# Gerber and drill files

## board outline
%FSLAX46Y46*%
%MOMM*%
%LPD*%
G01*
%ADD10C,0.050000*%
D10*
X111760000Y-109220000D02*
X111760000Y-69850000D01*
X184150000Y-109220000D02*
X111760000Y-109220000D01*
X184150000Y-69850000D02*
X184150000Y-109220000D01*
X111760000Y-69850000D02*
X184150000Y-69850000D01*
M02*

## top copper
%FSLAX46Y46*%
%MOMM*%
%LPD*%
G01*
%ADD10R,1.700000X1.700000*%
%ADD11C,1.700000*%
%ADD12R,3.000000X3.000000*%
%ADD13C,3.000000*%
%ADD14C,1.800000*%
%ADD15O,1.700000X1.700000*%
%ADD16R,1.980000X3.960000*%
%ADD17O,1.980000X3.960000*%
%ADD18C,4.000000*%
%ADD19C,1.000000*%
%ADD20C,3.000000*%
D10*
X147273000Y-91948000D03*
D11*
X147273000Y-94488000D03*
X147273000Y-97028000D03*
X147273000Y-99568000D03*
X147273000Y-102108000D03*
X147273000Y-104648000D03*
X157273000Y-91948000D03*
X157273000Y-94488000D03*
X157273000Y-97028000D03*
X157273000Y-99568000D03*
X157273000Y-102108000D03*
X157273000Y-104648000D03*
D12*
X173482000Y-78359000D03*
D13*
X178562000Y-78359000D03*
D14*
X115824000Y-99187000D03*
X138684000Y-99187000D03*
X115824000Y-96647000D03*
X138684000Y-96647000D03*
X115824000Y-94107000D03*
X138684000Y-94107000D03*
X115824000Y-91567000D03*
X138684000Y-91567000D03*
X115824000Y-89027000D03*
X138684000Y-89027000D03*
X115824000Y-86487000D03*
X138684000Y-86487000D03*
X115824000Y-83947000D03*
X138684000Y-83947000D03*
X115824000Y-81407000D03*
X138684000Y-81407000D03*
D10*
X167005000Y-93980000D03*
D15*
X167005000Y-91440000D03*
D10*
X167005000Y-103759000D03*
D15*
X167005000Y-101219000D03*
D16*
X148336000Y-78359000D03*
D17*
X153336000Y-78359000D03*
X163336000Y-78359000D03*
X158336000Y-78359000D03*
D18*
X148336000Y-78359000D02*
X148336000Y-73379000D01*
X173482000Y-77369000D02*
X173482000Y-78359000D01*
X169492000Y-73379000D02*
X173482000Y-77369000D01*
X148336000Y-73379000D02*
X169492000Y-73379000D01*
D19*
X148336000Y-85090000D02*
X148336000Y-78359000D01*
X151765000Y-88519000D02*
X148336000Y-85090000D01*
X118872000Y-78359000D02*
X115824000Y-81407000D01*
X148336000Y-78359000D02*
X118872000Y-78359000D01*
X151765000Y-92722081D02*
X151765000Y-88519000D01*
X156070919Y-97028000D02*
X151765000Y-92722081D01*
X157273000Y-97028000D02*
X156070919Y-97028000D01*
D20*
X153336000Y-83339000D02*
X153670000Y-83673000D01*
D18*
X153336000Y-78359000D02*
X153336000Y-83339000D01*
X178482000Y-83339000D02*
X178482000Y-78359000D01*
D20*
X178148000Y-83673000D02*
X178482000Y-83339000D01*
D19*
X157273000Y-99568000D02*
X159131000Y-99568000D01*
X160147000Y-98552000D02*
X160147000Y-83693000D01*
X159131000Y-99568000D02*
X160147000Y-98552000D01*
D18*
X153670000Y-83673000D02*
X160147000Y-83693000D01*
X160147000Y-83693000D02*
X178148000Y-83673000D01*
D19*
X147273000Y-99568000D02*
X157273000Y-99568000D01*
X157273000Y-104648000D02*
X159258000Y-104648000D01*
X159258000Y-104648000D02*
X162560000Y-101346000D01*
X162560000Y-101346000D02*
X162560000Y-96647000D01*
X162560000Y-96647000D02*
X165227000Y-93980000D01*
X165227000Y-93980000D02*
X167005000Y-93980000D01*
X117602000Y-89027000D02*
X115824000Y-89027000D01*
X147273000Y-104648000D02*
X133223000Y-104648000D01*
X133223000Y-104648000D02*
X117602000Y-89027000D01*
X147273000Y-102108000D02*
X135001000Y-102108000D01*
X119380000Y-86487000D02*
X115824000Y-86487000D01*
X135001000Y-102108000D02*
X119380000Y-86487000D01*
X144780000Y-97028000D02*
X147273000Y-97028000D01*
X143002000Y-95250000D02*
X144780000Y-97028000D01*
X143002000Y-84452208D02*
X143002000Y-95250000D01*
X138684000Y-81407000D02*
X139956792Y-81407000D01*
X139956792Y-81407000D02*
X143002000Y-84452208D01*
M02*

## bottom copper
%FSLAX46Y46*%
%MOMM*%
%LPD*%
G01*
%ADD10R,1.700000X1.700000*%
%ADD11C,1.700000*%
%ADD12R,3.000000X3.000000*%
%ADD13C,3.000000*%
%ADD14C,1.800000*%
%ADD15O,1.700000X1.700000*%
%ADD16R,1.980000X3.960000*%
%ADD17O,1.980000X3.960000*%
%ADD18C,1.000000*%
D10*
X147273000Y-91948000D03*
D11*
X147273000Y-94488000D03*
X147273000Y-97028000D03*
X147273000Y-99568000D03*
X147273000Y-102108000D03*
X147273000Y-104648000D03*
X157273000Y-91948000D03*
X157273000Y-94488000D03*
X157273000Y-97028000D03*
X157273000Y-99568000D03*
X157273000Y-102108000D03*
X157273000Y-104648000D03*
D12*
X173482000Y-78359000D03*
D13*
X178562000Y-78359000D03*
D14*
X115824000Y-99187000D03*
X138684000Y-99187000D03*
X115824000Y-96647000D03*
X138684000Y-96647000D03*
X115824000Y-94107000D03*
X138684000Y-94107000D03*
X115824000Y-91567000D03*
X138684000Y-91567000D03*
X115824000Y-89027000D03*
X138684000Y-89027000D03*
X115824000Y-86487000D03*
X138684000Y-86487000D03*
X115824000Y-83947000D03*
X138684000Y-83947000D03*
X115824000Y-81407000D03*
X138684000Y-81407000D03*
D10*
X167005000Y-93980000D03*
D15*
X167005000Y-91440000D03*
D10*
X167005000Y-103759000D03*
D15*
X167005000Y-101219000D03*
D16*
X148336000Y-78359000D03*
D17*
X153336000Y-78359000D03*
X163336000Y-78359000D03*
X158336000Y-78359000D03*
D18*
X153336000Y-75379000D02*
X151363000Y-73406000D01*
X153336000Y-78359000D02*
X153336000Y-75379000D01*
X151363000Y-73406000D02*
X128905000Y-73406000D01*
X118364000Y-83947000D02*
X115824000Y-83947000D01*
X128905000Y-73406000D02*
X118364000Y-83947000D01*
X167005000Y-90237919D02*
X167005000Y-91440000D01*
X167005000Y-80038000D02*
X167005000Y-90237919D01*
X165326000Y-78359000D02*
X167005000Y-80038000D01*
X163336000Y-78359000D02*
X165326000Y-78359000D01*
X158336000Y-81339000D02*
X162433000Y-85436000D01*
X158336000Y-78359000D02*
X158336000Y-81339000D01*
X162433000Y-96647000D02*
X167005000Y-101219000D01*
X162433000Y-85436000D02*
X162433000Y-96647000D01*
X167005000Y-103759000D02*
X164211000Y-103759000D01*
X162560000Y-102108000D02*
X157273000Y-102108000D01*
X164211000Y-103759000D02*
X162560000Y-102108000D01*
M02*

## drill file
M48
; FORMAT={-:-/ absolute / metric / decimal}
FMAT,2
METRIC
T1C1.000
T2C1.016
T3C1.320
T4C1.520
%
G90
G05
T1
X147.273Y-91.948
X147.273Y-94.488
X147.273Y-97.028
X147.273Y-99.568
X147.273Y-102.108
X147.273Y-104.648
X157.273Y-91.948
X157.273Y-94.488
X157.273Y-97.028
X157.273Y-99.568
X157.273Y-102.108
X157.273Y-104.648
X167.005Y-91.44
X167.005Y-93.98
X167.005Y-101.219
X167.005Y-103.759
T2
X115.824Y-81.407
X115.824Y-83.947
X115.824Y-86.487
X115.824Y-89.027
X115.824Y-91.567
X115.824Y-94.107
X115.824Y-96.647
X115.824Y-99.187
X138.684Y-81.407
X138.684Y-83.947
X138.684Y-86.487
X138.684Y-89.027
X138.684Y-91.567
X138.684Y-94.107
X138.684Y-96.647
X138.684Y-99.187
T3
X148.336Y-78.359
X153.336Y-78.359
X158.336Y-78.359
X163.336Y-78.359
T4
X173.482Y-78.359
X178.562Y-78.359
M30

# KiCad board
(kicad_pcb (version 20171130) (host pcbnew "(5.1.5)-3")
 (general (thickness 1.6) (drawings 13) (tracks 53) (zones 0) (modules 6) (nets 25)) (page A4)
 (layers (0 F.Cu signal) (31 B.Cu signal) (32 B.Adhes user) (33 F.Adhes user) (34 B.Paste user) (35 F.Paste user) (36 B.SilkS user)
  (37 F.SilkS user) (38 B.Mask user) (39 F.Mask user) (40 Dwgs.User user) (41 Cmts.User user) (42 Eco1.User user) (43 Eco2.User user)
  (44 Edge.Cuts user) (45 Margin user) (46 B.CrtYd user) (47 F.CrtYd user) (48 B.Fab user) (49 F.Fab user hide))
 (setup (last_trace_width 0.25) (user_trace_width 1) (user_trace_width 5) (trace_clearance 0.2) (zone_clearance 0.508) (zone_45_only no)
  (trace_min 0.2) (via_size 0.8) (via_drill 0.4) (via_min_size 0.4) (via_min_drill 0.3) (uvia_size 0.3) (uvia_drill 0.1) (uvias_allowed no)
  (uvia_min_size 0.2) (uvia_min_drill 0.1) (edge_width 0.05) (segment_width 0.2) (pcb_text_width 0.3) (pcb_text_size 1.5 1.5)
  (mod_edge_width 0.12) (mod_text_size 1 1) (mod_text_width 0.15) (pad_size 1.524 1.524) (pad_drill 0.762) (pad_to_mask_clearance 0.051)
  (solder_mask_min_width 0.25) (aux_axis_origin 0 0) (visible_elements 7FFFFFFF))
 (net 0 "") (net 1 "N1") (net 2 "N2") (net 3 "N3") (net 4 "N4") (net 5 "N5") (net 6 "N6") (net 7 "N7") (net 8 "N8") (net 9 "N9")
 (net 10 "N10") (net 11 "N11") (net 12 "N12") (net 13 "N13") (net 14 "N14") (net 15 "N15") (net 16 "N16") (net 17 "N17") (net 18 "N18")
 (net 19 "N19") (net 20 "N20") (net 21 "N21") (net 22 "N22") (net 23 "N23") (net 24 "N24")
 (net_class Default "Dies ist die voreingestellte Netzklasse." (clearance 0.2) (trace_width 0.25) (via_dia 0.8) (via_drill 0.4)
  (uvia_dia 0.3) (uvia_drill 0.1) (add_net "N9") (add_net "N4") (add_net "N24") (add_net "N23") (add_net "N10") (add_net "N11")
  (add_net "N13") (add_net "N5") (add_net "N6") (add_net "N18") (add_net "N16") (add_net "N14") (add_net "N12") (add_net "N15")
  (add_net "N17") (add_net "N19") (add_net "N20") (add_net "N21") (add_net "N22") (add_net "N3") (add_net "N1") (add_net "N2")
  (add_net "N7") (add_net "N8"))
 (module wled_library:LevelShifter (layer F.Cu) (at 152.273 98.298)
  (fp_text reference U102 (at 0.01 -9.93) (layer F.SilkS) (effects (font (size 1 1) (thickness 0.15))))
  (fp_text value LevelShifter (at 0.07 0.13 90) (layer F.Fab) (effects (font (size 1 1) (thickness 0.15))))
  (pad 1 thru_hole rect (at -5 -6.35) (size 1.7 1.7) (drill 1) (layers *.Cu *.Mask) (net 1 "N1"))
  (pad 2 thru_hole circle (at -5 -3.81) (size 1.7 1.7) (drill 1) (layers *.Cu *.Mask) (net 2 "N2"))
  (pad 3 thru_hole circle (at -5 -1.27) (size 1.7 1.7) (drill 1) (layers *.Cu *.Mask) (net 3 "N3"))
  (pad 4 thru_hole circle (at -5 1.27) (size 1.7 1.7) (drill 1) (layers *.Cu *.Mask) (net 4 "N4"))
  (pad 5 thru_hole circle (at -5 3.81) (size 1.7 1.7) (drill 1) (layers *.Cu *.Mask) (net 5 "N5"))
  (pad 6 thru_hole circle (at -5 6.35) (size 1.7 1.7) (drill 1) (layers *.Cu *.Mask) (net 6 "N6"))
  (pad 7 thru_hole circle (at 5 -6.35) (size 1.7 1.7) (drill 1) (layers *.Cu *.Mask) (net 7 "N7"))
  (pad 8 thru_hole circle (at 5 -3.81) (size 1.7 1.7) (drill 1) (layers *.Cu *.Mask) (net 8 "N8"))
  (pad 9 thru_hole circle (at 5 -1.27) (size 1.7 1.7) (drill 1) (layers *.Cu *.Mask) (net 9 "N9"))
  (pad 10 thru_hole circle (at 5 1.27) (size 1.7 1.7) (drill 1) (layers *.Cu *.Mask) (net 4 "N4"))
  (pad 11 thru_hole circle (at 5 3.81) (size 1.7 1.7) (drill 1) (layers *.Cu *.Mask) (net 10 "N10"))
  (pad 12 thru_hole circle (at 5 6.35) (size 1.7 1.7) (drill 1) (layers *.Cu *.Mask) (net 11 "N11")))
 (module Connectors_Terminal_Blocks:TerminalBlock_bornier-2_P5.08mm (layer F.Cu) (at 173.482 78.359)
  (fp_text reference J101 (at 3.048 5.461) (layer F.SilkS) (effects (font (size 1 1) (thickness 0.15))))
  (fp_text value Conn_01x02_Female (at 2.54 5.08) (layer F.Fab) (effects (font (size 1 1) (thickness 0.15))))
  (pad 1 thru_hole rect (at 0 0) (size 3 3) (drill 1.52) (layers *.Cu *.Mask) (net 9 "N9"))
  (pad 2 thru_hole circle (at 5.08 0) (size 3 3) (drill 1.52) (layers *.Cu *.Mask) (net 4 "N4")))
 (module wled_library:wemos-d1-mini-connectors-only (layer F.Cu) (at 127.254 90.297 270)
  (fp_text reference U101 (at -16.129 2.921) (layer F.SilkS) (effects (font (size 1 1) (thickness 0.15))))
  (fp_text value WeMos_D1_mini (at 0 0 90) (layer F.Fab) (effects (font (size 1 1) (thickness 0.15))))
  (pad 16 thru_hole circle (at 8.89 11.43 270) (size 1.8 1.8) (drill 1.016) (layers *.Cu *.Mask) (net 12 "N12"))
  (pad 1 thru_hole circle (at 8.89 -11.43 270) (size 1.8 1.8) (drill 1.016) (layers *.Cu *.Mask) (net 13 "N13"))
  (pad 15 thru_hole circle (at 6.35 11.43 270) (size 1.8 1.8) (drill 1.016) (layers *.Cu *.Mask) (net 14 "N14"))
  (pad 2 thru_hole circle (at 6.35 -11.43 270) (size 1.8 1.8) (drill 1.016) (layers *.Cu *.Mask) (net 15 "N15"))
  (pad 14 thru_hole circle (at 3.81 11.43 270) (size 1.8 1.8) (drill 1.016) (layers *.Cu *.Mask) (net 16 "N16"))
  (pad 3 thru_hole circle (at 3.81 -11.43 270) (size 1.8 1.8) (drill 1.016) (layers *.Cu *.Mask) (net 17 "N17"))
  (pad 13 thru_hole circle (at 1.27 11.43 270) (size 1.8 1.8) (drill 1.016) (layers *.Cu *.Mask) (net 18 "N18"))
  (pad 4 thru_hole circle (at 1.27 -11.43 270) (size 1.8 1.8) (drill 1.016) (layers *.Cu *.Mask) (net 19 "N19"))
  (pad 12 thru_hole circle (at -1.27 11.43 270) (size 1.8 1.8) (drill 1.016) (layers *.Cu *.Mask) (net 6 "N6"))
  (pad 5 thru_hole circle (at -1.27 -11.43 270) (size 1.8 1.8) (drill 1.016) (layers *.Cu *.Mask) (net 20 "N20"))
  (pad 11 thru_hole circle (at -3.81 11.43 270) (size 1.8 1.8) (drill 1.016) (layers *.Cu *.Mask) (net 5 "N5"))
  (pad 6 thru_hole circle (at -3.81 -11.43 270) (size 1.8 1.8) (drill 1.016) (layers *.Cu *.Mask) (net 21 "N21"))
  (pad 10 thru_hole circle (at -6.35 11.43 270) (size 1.8 1.8) (drill 1.016) (layers *.Cu *.Mask) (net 4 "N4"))
  (pad 7 thru_hole circle (at -6.35 -11.43 270) (size 1.8 1.8) (drill 1.016) (layers *.Cu *.Mask) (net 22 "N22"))
  (pad 9 thru_hole circle (at -8.89 11.43 270) (size 1.8 1.8) (drill 1.016) (layers *.Cu *.Mask) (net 9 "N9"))
  (pad 8 thru_hole circle (at -8.89 -11.43 270) (size 1.8 1.8) (drill 1.016) (layers *.Cu *.Mask) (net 3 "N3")))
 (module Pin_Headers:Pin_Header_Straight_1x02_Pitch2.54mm (layer F.Cu) (at 167.005 93.98 180)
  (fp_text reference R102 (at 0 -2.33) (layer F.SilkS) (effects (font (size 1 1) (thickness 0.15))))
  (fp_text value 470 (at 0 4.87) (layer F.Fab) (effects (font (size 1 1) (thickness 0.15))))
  (pad 1 thru_hole rect (at 0 0 180) (size 1.7 1.7) (drill 1) (layers *.Cu *.Mask) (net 11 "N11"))
  (pad 2 thru_hole oval (at 0 2.54 180) (size 1.7 1.7) (drill 1) (layers *.Cu *.Mask) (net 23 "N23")))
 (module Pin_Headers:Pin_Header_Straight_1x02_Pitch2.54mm (layer F.Cu) (at 167.005 103.759 180)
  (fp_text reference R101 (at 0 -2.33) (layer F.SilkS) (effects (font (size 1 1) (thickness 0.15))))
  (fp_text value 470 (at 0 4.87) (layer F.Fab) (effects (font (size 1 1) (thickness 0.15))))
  (pad 1 thru_hole rect (at 0 0 180) (size 1.7 1.7) (drill 1) (layers *.Cu *.Mask) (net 10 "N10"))
  (pad 2 thru_hole oval (at 0 2.54 180) (size 1.7 1.7) (drill 1) (layers *.Cu *.Mask) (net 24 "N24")))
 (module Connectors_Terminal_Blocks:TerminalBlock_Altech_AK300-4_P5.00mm (layer F.Cu) (at 148.336 78.359)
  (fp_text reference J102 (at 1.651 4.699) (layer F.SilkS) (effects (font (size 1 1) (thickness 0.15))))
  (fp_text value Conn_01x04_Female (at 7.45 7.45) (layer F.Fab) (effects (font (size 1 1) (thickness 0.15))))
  (pad 1 thru_hole rect (at 0 0) (size 1.98 3.96) (drill 1.32) (layers *.Cu *.Mask) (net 9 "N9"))
  (pad 2 thru_hole oval (at 5 0) (size 1.98 3.96) (drill 1.32) (layers *.Cu *.Mask) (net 4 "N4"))
  (pad 4 thru_hole oval (at 15 0) (size 1.98 3.96) (drill 1.32) (layers *.Cu *.Mask) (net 23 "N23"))
  (pad 3 thru_hole oval (at 10 0) (size 1.98 3.96) (drill 1.32) (layers *.Cu *.Mask) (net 24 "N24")))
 (gr_line (start 111.76 109.22) (end 111.76 69.85) (layer Edge.Cuts) (width 0.05))
 (gr_line (start 184.15 109.22) (end 111.76 109.22) (layer Edge.Cuts) (width 0.05))
 (gr_line (start 184.15 69.85) (end 184.15 109.22) (layer Edge.Cuts) (width 0.05))
 (gr_line (start 111.76 69.85) (end 184.15 69.85) (layer Edge.Cuts) (width 0.05))
 (segment (start 148.336 78.359) (end 148.336 73.379) (width 4) (layer F.Cu) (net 9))
 (segment (start 173.482 77.369) (end 173.482 78.359) (width 4) (layer F.Cu) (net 9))
 (segment (start 169.492 73.379) (end 173.482 77.369) (width 4) (layer F.Cu) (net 9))
 (segment (start 148.336 73.379) (end 169.492 73.379) (width 4) (layer F.Cu) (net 9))
 (segment (start 148.336 85.09) (end 148.336 78.359) (width 1) (layer F.Cu) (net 9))
 (segment (start 151.765 88.519) (end 148.336 85.09) (width 1) (layer F.Cu) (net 9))
 (segment (start 118.872 78.359) (end 115.824 81.407) (width 1) (layer F.Cu) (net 9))
 (segment (start 148.336 78.359) (end 118.872 78.359) (width 1) (layer F.Cu) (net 9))
 (segment (start 151.765 92.722081) (end 151.765 88.519) (width 1) (layer F.Cu) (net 9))
 (segment (start 156.070919 97.028) (end 151.765 92.722081) (width 1) (layer F.Cu) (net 9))
 (segment (start 157.273 97.028) (end 156.070919 97.028) (width 1) (layer F.Cu) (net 9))
 (segment (start 153.336 83.339) (end 153.67 83.673) (width 3) (layer F.Cu) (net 4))
 (segment (start 153.336 78.359) (end 153.336 83.339) (width 4) (layer F.Cu) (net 4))
 (segment (start 178.482 83.339) (end 178.482 78.359) (width 4) (layer F.Cu) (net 4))
 (segment (start 178.148 83.673) (end 178.482 83.339) (width 3) (layer F.Cu) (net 4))
 (segment (start 157.273 99.568) (end 159.131 99.568) (width 1) (layer F.Cu) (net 4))
 (segment (start 160.147 98.552) (end 160.147 83.693) (width 1) (layer F.Cu) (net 4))
 (segment (start 159.131 99.568) (end 160.147 98.552) (width 1) (layer F.Cu) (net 4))
 (segment (start 153.67 83.673) (end 160.147 83.693) (width 4) (layer F.Cu) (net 4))
 (segment (start 160.147 83.693) (end 178.148 83.673) (width 4) (layer F.Cu) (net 4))
 (segment (start 153.336 75.379) (end 151.363 73.406) (width 1) (layer B.Cu) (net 4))
 (segment (start 153.336 78.359) (end 153.336 75.379) (width 1) (layer B.Cu) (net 4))
 (segment (start 151.363 73.406) (end 128.905 73.406) (width 1) (layer B.Cu) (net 4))
 (segment (start 118.364 83.947) (end 115.824 83.947) (width 1) (layer B.Cu) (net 4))
 (segment (start 128.905 73.406) (end 118.364 83.947) (width 1) (layer B.Cu) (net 4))
 (segment (start 147.273 99.568) (end 157.273 99.568) (width 1) (layer F.Cu) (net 4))
 (segment (start 167.005 90.237919) (end 167.005 91.44) (width 1) (layer B.Cu) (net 23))
 (segment (start 167.005 80.038) (end 167.005 90.237919) (width 1) (layer B.Cu) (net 23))
 (segment (start 165.326 78.359) (end 167.005 80.038) (width 1) (layer B.Cu) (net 23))
 (segment (start 163.336 78.359) (end 165.326 78.359) (width 1) (layer B.Cu) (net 23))
 (segment (start 158.336 81.339) (end 162.433 85.436) (width 1) (layer B.Cu) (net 24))
 (segment (start 158.336 78.359) (end 158.336 81.339) (width 1) (layer B.Cu) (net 24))
 (segment (start 162.433 96.647) (end 167.005 101.219) (width 1) (layer B.Cu) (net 24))
 (segment (start 162.433 85.436) (end 162.433 96.647) (width 1) (layer B.Cu) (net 24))
 (segment (start 167.005 103.759) (end 164.211 103.759) (width 1) (layer B.Cu) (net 10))
 (segment (start 162.56 102.108) (end 157.273 102.108) (width 1) (layer B.Cu) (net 10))
 (segment (start 164.211 103.759) (end 162.56 102.108) (width 1) (layer B.Cu) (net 10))
 (segment (start 157.273 104.648) (end 159.258 104.648) (width 1) (layer F.Cu) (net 11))
 (segment (start 159.258 104.648) (end 162.56 101.346) (width 1) (layer F.Cu) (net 11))
 (segment (start 162.56 101.346) (end 162.56 96.647) (width 1) (layer F.Cu) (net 11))
 (segment (start 162.56 96.647) (end 165.227 93.98) (width 1) (layer F.Cu) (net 11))
 (segment (start 165.227 93.98) (end 167.005 93.98) (width 1) (layer F.Cu) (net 11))
 (segment (start 117.602 89.027) (end 115.824 89.027) (width 1) (layer F.Cu) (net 6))
 (segment (start 147.273 104.648) (end 133.223 104.648) (width 1) (layer F.Cu) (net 6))
 (segment (start 133.223 104.648) (end 117.602 89.027) (width 1) (layer F.Cu) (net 6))
 (segment (start 147.273 102.108) (end 135.001 102.108) (width 1) (layer F.Cu) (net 5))
 (segment (start 119.38 86.487) (end 115.824 86.487) (width 1) (layer F.Cu) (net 5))
 (segment (start 135.001 102.108) (end 119.38 86.487) (width 1) (layer F.Cu) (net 5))
 (segment (start 144.78 97.028) (end 147.273 97.028) (width 1) (layer F.Cu) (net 3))
 (segment (start 143.002 95.25) (end 144.78 97.028) (width 1) (layer F.Cu) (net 3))
 (segment (start 143.002 84.452208) (end 143.002 95.25) (width 1) (layer F.Cu) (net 3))
 (segment (start 138.684 81.407) (end 139.956792 81.407) (width 1) (layer F.Cu) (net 3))
 (segment (start 139.956792 81.407) (end 143.002 84.452208) (width 1) (layer F.Cu) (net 3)))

